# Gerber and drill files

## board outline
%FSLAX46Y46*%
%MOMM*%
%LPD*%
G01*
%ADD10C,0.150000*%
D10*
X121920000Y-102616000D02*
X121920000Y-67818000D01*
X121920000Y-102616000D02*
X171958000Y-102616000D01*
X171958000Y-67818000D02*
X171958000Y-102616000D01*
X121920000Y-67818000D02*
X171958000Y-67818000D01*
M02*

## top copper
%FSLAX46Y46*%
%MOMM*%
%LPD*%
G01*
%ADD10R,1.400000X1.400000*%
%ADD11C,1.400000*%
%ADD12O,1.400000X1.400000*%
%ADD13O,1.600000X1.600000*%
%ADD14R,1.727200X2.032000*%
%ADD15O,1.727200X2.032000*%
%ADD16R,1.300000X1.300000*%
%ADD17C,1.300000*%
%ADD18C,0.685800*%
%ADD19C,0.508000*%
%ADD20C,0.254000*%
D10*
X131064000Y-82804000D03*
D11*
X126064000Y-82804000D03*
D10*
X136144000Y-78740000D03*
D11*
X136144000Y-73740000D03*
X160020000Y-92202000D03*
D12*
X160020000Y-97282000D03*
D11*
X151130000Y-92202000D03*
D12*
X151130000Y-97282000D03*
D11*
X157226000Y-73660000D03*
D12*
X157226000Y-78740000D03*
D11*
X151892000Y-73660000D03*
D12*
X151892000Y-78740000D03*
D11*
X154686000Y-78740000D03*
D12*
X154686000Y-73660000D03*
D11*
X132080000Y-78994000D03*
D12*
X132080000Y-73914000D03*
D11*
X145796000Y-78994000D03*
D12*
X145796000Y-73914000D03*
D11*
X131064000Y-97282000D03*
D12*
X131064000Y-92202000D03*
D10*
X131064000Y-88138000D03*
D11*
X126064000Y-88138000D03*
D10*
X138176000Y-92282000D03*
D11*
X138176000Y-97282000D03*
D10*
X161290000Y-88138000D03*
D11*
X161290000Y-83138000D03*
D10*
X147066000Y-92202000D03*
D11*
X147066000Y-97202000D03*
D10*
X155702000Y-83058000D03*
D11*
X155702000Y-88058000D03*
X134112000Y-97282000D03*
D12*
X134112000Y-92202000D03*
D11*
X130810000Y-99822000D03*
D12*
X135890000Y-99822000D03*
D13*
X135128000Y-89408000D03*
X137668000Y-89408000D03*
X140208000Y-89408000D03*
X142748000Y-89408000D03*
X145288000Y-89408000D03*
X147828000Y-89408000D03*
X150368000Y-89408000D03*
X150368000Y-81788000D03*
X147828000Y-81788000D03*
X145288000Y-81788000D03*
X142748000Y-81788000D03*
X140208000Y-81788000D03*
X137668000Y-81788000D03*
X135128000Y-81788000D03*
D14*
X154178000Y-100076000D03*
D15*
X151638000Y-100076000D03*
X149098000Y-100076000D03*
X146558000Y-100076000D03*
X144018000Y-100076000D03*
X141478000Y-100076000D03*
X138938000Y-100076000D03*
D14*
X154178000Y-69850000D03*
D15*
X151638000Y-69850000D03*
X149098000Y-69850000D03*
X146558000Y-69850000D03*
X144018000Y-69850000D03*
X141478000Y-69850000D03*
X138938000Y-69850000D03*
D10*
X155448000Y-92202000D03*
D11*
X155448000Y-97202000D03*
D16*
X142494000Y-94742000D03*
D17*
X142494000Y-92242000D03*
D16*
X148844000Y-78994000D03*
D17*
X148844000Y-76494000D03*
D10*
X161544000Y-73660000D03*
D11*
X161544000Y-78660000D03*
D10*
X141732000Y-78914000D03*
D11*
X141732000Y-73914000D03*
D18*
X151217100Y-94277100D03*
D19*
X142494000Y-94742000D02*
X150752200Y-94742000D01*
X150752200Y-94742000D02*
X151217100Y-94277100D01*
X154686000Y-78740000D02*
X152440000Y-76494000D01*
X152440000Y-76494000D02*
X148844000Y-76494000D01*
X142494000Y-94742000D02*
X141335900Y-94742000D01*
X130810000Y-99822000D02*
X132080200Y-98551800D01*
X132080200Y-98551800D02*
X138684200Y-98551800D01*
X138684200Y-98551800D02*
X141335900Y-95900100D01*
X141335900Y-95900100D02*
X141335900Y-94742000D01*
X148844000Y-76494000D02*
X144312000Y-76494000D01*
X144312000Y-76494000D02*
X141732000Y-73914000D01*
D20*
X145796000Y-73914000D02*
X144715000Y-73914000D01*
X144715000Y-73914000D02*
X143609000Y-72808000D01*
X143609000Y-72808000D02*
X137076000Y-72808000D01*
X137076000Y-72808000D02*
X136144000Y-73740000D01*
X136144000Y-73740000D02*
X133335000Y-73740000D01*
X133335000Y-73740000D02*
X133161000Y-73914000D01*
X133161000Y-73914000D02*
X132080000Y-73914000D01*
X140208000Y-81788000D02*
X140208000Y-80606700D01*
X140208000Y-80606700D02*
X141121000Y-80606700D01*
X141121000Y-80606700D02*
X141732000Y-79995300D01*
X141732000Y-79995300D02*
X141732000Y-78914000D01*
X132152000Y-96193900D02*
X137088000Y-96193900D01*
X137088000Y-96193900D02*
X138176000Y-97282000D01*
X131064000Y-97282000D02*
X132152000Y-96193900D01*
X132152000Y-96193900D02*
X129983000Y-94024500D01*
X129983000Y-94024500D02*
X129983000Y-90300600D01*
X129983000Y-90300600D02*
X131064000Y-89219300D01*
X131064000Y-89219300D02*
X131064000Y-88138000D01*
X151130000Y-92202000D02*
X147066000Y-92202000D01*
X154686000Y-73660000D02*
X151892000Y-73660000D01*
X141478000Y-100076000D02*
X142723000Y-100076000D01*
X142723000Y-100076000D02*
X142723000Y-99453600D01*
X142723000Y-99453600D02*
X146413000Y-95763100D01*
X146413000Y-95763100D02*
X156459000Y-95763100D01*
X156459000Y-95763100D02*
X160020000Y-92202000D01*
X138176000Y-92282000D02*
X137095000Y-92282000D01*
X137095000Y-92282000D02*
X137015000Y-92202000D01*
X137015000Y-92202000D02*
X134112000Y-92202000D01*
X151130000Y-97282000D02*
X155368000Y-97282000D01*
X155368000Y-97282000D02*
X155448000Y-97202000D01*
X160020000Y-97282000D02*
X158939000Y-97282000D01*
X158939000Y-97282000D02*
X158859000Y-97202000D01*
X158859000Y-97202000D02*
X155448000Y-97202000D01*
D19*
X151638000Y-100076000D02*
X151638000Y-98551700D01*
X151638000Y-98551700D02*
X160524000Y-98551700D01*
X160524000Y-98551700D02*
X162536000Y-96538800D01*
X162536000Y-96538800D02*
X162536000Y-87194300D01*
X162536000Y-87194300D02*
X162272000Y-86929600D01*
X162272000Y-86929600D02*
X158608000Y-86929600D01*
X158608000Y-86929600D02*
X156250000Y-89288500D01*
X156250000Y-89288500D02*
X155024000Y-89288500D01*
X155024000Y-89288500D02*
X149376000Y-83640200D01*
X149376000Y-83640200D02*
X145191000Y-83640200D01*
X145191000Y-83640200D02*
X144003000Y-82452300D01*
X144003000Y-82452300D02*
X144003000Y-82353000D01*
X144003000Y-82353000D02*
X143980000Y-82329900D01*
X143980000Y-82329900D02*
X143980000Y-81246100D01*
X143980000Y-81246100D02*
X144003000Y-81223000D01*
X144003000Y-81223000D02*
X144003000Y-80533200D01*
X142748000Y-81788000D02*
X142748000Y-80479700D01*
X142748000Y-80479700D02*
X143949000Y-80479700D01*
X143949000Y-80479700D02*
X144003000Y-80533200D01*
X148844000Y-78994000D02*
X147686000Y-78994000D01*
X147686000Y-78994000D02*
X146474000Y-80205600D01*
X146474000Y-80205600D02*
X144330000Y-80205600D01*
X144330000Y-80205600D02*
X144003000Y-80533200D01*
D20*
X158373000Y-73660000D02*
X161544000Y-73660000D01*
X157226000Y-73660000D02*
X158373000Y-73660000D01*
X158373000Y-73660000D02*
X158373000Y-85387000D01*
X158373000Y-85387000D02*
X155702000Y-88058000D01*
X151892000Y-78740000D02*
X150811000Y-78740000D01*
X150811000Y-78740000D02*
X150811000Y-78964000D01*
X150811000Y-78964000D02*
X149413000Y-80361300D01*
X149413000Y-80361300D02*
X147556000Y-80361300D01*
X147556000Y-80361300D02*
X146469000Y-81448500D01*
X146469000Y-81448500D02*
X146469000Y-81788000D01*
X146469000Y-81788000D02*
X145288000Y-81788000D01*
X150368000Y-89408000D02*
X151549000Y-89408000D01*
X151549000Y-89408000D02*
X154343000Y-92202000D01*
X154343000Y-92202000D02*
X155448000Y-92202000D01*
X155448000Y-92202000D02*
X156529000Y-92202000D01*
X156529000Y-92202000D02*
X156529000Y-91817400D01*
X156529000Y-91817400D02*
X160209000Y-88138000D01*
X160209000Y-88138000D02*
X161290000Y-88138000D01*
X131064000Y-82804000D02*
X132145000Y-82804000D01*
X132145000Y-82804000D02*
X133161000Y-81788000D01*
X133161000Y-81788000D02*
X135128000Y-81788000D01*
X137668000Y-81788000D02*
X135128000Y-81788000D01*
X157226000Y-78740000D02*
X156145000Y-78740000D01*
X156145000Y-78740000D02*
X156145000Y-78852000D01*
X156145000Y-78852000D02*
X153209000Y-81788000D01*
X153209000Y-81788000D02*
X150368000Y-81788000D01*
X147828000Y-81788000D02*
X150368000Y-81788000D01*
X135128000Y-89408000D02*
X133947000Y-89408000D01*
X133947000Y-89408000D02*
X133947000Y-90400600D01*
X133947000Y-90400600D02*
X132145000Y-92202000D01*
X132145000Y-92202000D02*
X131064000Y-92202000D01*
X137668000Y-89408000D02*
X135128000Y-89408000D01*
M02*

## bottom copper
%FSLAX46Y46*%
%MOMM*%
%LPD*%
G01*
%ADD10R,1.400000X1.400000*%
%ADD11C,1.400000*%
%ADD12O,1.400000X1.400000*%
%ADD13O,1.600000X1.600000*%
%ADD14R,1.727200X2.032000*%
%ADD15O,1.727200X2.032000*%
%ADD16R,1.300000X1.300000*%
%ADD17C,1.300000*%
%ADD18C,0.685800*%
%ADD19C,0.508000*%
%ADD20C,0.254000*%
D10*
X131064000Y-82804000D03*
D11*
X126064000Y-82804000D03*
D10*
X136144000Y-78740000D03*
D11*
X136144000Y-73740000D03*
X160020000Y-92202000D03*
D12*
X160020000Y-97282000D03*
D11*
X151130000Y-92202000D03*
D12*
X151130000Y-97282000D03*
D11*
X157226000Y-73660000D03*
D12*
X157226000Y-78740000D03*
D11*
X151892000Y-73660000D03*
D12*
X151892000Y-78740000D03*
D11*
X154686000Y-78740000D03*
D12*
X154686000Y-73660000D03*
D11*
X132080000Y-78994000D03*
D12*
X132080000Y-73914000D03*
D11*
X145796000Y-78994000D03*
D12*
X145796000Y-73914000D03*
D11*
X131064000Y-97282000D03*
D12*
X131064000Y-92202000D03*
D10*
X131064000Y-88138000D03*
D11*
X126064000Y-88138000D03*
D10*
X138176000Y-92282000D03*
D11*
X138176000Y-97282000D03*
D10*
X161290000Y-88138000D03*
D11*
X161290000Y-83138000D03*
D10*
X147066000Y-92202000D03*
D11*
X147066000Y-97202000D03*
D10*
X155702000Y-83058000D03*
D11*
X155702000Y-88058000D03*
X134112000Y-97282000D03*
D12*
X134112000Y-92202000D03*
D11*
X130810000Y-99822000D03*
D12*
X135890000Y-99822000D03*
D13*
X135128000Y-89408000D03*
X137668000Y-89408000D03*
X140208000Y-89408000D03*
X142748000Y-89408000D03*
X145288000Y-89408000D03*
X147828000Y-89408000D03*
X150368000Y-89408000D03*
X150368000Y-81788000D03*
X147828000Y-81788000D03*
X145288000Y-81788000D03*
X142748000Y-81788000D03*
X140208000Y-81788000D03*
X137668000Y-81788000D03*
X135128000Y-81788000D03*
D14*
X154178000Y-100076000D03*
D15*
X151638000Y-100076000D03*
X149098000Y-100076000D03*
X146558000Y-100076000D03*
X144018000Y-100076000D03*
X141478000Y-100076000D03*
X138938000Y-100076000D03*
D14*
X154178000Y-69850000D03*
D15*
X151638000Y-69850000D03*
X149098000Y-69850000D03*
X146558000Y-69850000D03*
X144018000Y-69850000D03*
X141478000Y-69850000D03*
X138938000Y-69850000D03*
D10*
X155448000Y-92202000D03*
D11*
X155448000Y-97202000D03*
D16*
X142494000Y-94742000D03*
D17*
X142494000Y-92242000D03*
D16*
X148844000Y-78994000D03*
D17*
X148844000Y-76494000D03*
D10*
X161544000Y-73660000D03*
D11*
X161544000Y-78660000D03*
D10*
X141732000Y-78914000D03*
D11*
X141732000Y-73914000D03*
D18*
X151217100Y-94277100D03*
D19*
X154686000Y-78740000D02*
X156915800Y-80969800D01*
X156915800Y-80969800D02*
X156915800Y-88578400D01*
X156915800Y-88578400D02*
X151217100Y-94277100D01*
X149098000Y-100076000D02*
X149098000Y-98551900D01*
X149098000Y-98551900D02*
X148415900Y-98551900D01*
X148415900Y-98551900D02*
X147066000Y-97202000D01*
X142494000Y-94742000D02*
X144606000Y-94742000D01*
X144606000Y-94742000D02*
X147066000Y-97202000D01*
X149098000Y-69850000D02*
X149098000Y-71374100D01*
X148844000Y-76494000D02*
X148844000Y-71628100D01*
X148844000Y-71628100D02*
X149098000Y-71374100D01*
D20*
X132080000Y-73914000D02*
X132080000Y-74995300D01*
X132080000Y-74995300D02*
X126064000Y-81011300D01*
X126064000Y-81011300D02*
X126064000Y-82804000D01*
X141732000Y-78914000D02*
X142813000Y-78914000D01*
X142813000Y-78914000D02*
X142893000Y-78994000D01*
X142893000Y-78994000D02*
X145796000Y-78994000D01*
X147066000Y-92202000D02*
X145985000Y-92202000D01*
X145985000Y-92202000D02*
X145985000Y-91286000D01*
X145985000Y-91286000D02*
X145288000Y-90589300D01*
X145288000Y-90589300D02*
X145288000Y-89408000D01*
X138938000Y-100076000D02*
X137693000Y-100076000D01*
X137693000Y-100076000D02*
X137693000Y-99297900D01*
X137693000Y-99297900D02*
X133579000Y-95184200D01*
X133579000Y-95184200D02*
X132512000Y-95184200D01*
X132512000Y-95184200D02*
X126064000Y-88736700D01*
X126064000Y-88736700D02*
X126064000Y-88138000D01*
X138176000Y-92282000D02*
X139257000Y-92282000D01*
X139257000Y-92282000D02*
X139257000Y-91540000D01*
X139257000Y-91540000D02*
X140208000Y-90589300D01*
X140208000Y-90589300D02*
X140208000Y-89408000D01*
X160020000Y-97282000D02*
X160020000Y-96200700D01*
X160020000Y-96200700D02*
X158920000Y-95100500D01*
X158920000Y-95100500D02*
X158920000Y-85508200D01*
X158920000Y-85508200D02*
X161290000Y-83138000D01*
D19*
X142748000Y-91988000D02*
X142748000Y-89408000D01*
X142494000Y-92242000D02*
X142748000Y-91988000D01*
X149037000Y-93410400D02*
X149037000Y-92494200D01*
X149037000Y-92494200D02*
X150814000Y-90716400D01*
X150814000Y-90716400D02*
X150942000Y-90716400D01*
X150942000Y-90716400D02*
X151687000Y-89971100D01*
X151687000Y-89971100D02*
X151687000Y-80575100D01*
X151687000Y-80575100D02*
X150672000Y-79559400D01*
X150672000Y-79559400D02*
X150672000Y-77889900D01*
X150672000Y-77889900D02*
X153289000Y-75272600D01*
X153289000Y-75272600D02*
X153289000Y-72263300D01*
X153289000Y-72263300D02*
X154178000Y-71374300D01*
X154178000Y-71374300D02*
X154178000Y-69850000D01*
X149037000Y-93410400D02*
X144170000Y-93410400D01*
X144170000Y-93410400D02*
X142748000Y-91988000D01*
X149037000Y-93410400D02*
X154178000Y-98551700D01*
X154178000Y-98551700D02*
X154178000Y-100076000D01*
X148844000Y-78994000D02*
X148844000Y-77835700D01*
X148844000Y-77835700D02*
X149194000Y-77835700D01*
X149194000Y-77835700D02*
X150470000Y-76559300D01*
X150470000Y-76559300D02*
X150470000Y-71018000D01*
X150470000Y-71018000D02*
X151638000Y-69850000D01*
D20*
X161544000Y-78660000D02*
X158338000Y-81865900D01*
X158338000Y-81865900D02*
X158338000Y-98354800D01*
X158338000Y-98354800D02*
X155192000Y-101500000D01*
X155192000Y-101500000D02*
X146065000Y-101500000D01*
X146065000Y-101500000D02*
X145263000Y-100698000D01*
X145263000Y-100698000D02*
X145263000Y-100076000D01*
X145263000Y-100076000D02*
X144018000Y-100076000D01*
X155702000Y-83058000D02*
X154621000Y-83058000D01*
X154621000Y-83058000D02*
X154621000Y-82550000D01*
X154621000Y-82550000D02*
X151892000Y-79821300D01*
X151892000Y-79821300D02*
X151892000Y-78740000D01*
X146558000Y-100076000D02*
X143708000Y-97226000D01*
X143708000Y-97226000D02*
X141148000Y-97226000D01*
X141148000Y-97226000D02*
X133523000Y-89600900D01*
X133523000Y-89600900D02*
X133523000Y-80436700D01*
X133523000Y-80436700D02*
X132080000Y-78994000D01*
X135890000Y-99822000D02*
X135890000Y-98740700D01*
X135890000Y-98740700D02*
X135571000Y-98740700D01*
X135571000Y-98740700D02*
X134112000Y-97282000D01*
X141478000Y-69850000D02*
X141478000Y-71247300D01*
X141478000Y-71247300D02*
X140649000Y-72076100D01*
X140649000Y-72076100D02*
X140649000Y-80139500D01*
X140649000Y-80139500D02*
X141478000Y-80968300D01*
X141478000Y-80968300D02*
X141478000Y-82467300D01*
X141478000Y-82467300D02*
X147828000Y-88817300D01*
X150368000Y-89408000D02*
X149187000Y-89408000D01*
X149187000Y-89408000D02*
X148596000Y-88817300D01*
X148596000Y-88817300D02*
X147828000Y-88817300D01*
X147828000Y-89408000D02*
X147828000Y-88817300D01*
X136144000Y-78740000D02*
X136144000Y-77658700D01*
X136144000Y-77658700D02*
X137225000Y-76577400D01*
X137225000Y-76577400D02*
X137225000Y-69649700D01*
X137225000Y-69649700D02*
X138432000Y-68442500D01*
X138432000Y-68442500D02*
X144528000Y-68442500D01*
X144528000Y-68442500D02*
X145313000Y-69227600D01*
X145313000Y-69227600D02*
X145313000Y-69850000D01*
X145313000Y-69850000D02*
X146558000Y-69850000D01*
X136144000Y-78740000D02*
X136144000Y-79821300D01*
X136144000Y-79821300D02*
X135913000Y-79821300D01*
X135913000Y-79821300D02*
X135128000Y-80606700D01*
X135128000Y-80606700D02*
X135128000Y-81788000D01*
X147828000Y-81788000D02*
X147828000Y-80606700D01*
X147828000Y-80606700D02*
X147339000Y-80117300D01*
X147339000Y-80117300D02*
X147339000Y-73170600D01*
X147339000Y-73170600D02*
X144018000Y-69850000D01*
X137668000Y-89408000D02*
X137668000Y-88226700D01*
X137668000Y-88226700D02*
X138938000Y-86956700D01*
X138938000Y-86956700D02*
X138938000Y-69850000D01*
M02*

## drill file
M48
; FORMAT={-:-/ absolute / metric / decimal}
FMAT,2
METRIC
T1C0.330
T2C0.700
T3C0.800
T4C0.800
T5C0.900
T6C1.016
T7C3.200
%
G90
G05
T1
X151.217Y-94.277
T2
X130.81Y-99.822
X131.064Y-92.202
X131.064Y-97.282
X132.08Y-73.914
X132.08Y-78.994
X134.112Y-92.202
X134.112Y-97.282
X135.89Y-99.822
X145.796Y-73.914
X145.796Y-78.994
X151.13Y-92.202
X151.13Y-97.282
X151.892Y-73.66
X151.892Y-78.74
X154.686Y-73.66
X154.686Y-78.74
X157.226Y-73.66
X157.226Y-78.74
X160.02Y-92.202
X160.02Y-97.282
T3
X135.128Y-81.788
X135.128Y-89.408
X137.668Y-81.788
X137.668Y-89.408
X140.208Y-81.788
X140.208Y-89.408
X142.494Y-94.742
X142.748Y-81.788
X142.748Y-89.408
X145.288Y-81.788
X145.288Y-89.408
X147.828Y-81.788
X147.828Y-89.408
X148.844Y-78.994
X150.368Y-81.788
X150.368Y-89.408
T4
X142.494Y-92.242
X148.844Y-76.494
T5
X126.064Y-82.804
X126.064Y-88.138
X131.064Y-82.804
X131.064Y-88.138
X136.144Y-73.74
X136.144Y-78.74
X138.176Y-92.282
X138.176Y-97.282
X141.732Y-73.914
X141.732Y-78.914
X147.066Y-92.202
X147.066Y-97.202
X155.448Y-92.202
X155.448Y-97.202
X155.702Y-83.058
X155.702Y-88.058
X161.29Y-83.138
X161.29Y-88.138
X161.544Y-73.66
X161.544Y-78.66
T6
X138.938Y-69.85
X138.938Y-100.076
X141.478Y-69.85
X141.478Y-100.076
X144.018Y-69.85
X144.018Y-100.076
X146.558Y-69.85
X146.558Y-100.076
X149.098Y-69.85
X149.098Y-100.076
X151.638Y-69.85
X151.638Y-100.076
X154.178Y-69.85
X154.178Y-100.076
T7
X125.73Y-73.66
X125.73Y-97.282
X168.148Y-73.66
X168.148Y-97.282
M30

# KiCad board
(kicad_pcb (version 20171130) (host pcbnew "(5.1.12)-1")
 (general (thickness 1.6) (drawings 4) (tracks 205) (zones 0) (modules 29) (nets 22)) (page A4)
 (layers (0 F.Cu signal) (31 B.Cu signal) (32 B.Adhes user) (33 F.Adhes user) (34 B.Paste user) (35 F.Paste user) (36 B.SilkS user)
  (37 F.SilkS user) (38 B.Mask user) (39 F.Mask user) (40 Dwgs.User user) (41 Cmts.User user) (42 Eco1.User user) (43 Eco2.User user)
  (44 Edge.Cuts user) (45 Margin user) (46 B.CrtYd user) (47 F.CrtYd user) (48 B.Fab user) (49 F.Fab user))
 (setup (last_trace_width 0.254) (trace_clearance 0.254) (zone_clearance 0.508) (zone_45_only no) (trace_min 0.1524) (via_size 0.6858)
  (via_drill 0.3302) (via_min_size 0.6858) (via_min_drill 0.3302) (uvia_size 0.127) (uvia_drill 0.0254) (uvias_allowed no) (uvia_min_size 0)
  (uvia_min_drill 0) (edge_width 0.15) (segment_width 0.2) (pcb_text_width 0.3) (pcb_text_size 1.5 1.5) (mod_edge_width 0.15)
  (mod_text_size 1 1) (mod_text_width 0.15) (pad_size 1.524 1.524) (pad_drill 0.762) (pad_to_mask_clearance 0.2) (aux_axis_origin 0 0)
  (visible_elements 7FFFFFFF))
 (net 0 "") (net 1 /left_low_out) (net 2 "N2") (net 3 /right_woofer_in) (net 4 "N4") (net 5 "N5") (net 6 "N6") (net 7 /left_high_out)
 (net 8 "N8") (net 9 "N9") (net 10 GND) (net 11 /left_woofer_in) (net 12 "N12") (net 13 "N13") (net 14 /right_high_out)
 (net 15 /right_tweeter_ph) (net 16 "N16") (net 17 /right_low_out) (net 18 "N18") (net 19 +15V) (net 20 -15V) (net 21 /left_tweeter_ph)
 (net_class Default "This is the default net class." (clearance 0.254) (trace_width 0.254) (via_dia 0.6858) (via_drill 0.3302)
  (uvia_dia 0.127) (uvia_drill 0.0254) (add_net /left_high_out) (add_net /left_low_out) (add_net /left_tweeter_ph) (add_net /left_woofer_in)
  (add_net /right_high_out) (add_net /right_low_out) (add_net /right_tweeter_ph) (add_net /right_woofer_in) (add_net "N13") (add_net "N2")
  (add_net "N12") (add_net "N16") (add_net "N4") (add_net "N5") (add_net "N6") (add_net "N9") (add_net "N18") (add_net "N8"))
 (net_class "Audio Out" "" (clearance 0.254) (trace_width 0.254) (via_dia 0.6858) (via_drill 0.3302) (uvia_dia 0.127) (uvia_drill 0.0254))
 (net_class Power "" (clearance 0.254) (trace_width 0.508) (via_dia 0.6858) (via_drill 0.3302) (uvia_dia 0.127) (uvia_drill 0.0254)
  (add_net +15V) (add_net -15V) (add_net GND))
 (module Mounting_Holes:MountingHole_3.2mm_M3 (layer F.Cu) (at 125.73 97.282)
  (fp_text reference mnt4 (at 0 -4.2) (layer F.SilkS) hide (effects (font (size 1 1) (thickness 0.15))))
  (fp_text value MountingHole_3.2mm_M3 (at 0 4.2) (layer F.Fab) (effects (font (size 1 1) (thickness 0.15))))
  (pad 1 np_thru_hole circle (at 0 0) (size 3.2 3.2) (drill 3.2) (layers *.Cu *.Mask)))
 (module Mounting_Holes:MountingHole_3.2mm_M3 (layer F.Cu) (at 125.73 73.66)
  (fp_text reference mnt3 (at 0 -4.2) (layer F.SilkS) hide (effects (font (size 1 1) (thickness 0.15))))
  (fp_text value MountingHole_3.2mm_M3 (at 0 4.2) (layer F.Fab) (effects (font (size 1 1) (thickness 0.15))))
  (pad 1 np_thru_hole circle (at 0 0) (size 3.2 3.2) (drill 3.2) (layers *.Cu *.Mask)))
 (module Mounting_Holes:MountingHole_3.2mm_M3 (layer F.Cu) (at 168.148 97.282)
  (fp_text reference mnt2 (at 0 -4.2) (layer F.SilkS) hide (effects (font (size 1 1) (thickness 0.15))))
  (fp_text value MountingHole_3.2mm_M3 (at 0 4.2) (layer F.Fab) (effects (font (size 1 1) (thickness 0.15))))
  (pad 1 np_thru_hole circle (at 0 0) (size 3.2 3.2) (drill 3.2) (layers *.Cu *.Mask)))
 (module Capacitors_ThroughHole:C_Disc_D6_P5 (layer F.Cu) (at 131.064 82.804 180)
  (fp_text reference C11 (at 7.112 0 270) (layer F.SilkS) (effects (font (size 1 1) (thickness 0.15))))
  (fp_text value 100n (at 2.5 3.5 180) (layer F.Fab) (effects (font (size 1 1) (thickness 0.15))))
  (pad 1 thru_hole rect (at 0 0 180) (size 1.4 1.4) (drill 0.9) (layers *.Cu *.Mask) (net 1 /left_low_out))
  (pad 2 thru_hole circle (at 5 0 180) (size 1.4 1.4) (drill 0.9) (layers *.Cu *.Mask) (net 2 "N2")))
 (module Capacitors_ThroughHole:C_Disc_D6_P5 (layer F.Cu) (at 136.144 78.74 90)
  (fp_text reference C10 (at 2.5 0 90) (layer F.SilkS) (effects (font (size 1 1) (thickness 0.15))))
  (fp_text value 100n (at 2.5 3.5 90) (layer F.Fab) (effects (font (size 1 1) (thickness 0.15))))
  (pad 1 thru_hole rect (at 0 0 90) (size 1.4 1.4) (drill 0.9) (layers *.Cu *.Mask) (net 1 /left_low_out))
  (pad 2 thru_hole circle (at 5 0 90) (size 1.4 1.4) (drill 0.9) (layers *.Cu *.Mask) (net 2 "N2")))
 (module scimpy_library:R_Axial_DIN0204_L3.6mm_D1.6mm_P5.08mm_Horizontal (layer F.Cu) (at 160.02 92.202 270)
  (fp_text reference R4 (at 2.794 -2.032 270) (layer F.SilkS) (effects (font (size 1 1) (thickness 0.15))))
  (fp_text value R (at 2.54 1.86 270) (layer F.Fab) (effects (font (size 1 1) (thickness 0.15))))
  (pad 1 thru_hole circle (at 0 0 270) (size 1.4 1.4) (drill 0.7) (layers *.Cu *.Mask) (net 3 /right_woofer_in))
  (pad 2 thru_hole oval (at 5.08 0 270) (size 1.4 1.4) (drill 0.7) (layers *.Cu *.Mask) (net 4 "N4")))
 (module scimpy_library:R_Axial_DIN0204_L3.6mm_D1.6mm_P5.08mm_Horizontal (layer F.Cu) (at 151.13 92.202 270)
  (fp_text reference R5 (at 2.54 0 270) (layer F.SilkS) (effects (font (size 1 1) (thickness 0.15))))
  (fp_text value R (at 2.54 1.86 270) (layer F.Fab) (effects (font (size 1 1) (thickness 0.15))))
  (pad 1 thru_hole circle (at 0 0 270) (size 1.4 1.4) (drill 0.7) (layers *.Cu *.Mask) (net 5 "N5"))
  (pad 2 thru_hole oval (at 5.08 0 270) (size 1.4 1.4) (drill 0.7) (layers *.Cu *.Mask) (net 4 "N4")))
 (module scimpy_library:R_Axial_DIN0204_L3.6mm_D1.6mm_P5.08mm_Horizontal (layer F.Cu) (at 157.226 73.66 270)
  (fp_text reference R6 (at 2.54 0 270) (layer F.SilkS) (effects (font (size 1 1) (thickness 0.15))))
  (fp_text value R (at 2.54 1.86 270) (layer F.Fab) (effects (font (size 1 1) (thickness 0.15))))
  (pad 1 thru_hole circle (at 0 0 270) (size 1.4 1.4) (drill 0.7) (layers *.Cu *.Mask) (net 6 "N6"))
  (pad 2 thru_hole oval (at 5.08 0 270) (size 1.4 1.4) (drill 0.7) (layers *.Cu *.Mask) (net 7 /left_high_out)))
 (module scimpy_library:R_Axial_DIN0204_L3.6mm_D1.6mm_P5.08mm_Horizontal (layer F.Cu) (at 151.892 73.66 270)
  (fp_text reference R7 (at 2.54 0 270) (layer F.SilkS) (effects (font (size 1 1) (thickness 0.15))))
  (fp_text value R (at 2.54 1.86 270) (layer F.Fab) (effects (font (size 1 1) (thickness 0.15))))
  (pad 1 thru_hole circle (at 0 0 270) (size 1.4 1.4) (drill 0.7) (layers *.Cu *.Mask) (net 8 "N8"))
  (pad 2 thru_hole oval (at 5.08 0 270) (size 1.4 1.4) (drill 0.7) (layers *.Cu *.Mask) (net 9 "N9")))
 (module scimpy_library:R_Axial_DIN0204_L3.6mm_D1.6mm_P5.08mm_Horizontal (layer F.Cu) (at 154.686 78.74 90)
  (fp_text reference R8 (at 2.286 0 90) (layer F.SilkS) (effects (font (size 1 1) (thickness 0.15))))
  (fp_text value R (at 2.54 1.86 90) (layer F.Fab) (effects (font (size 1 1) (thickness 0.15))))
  (pad 1 thru_hole circle (at 0 0 90) (size 1.4 1.4) (drill 0.7) (layers *.Cu *.Mask) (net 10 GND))
  (pad 2 thru_hole oval (at 5.08 0 90) (size 1.4 1.4) (drill 0.7) (layers *.Cu *.Mask) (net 8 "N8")))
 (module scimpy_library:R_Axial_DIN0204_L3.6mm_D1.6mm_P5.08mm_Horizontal (layer F.Cu) (at 132.08 78.994 90)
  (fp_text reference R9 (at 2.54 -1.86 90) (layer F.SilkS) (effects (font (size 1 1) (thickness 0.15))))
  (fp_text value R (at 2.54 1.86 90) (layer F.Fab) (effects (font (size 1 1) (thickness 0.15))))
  (pad 1 thru_hole circle (at 0 0 90) (size 1.4 1.4) (drill 0.7) (layers *.Cu *.Mask) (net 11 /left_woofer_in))
  (pad 2 thru_hole oval (at 5.08 0 90) (size 1.4 1.4) (drill 0.7) (layers *.Cu *.Mask) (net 2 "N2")))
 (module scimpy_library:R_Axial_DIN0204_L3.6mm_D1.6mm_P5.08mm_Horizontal (layer F.Cu) (at 145.796 78.994 90)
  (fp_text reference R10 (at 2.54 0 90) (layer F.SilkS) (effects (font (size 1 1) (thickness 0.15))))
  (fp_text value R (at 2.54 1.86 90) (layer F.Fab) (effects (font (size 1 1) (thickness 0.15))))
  (pad 1 thru_hole circle (at 0 0 90) (size 1.4 1.4) (drill 0.7) (layers *.Cu *.Mask) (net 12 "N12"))
  (pad 2 thru_hole oval (at 5.08 0 90) (size 1.4 1.4) (drill 0.7) (layers *.Cu *.Mask) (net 2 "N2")))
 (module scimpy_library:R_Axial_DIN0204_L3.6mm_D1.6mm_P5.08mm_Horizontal (layer F.Cu) (at 131.064 97.282 90)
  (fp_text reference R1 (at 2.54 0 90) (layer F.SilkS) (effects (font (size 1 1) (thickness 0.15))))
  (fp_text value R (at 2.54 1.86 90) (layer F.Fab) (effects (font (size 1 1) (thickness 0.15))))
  (pad 1 thru_hole circle (at 0 0 90) (size 1.4 1.4) (drill 0.7) (layers *.Cu *.Mask) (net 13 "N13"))
  (pad 2 thru_hole oval (at 5.08 0 90) (size 1.4 1.4) (drill 0.7) (layers *.Cu *.Mask) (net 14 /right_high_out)))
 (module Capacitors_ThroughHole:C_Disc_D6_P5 (layer F.Cu) (at 131.064 88.138 180)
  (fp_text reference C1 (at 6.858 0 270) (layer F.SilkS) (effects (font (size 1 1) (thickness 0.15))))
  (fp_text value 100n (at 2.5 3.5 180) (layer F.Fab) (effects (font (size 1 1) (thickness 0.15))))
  (pad 1 thru_hole rect (at 0 0 180) (size 1.4 1.4) (drill 0.9) (layers *.Cu *.Mask) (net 13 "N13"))
  (pad 2 thru_hole circle (at 5 0 180) (size 1.4 1.4) (drill 0.9) (layers *.Cu *.Mask) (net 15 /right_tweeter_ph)))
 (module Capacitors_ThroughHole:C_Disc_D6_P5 (layer F.Cu) (at 138.176 92.282 270)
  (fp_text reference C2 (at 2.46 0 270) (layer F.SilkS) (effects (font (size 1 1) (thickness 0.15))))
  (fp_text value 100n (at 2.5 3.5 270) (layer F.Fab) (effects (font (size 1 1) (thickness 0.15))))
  (pad 1 thru_hole rect (at 0 0 270) (size 1.4 1.4) (drill 0.9) (layers *.Cu *.Mask) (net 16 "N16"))
  (pad 2 thru_hole circle (at 5 0 270) (size 1.4 1.4) (drill 0.9) (layers *.Cu *.Mask) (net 13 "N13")))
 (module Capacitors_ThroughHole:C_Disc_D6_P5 (layer F.Cu) (at 161.29 88.138 90)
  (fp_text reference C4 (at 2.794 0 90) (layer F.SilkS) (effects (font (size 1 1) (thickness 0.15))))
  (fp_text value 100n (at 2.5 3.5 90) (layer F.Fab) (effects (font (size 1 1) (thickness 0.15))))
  (pad 1 thru_hole rect (at 0 0 90) (size 1.4 1.4) (drill 0.9) (layers *.Cu *.Mask) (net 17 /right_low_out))
  (pad 2 thru_hole circle (at 5 0 90) (size 1.4 1.4) (drill 0.9) (layers *.Cu *.Mask) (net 4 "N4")))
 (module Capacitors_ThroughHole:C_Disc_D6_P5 (layer F.Cu) (at 147.066 92.202 270)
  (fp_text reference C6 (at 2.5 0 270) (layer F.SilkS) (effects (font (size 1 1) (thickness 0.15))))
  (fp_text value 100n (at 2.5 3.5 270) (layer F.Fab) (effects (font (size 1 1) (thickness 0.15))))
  (pad 1 thru_hole rect (at 0 0 270) (size 1.4 1.4) (drill 0.9) (layers *.Cu *.Mask) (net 5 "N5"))
  (pad 2 thru_hole circle (at 5 0 270) (size 1.4 1.4) (drill 0.9) (layers *.Cu *.Mask) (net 10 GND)))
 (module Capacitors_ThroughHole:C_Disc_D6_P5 (layer F.Cu) (at 155.702 83.058 270)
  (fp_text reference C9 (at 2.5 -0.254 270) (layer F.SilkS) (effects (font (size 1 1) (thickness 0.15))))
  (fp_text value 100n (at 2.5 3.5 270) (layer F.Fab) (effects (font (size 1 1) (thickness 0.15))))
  (pad 1 thru_hole rect (at 0 0 270) (size 1.4 1.4) (drill 0.9) (layers *.Cu *.Mask) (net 9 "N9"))
  (pad 2 thru_hole circle (at 5 0 270) (size 1.4 1.4) (drill 0.9) (layers *.Cu *.Mask) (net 6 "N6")))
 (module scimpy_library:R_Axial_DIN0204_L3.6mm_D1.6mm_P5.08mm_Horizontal (layer F.Cu) (at 134.112 97.282 90)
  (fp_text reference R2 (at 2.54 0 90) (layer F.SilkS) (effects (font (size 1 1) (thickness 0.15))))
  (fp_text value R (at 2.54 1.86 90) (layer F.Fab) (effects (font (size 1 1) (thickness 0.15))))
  (pad 1 thru_hole circle (at 0 0 90) (size 1.4 1.4) (drill 0.7) (layers *.Cu *.Mask) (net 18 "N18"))
  (pad 2 thru_hole oval (at 5.08 0 90) (size 1.4 1.4) (drill 0.7) (layers *.Cu *.Mask) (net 16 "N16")))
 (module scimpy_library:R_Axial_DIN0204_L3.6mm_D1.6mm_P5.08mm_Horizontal (layer F.Cu) (at 130.81 99.822)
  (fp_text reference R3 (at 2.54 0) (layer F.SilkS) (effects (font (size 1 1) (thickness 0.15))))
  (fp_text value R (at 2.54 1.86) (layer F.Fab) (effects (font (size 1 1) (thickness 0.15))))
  (pad 1 thru_hole circle (at 0 0) (size 1.4 1.4) (drill 0.7) (layers *.Cu *.Mask) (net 10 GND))
  (pad 2 thru_hole oval (at 5.08 0) (size 1.4 1.4) (drill 0.7) (layers *.Cu *.Mask) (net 18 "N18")))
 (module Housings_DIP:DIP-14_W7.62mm (layer F.Cu) (at 135.128 89.408 90)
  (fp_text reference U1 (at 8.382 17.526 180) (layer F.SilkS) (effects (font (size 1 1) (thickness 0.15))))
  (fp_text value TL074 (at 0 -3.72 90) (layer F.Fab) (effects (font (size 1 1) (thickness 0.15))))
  (pad 1 thru_hole oval (at 0 0 90) (size 1.6 1.6) (drill 0.8) (layers *.Cu *.Mask) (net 14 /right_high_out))
  (pad 2 thru_hole oval (at 0 2.54 90) (size 1.6 1.6) (drill 0.8) (layers *.Cu *.Mask) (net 14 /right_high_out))
  (pad 3 thru_hole oval (at 0 5.08 90) (size 1.6 1.6) (drill 0.8) (layers *.Cu *.Mask) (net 16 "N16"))
  (pad 4 thru_hole oval (at 0 7.62 90) (size 1.6 1.6) (drill 0.8) (layers *.Cu *.Mask) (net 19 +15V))
  (pad 5 thru_hole oval (at 0 10.16 90) (size 1.6 1.6) (drill 0.8) (layers *.Cu *.Mask) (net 5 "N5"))
  (pad 6 thru_hole oval (at 0 12.7 90) (size 1.6 1.6) (drill 0.8) (layers *.Cu *.Mask) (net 17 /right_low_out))
  (pad 7 thru_hole oval (at 0 15.24 90) (size 1.6 1.6) (drill 0.8) (layers *.Cu *.Mask) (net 17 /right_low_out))
  (pad 8 thru_hole oval (at 7.62 15.24 90) (size 1.6 1.6) (drill 0.8) (layers *.Cu *.Mask) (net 7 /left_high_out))
  (pad 9 thru_hole oval (at 7.62 12.7 90) (size 1.6 1.6) (drill 0.8) (layers *.Cu *.Mask) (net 7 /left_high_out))
  (pad 10 thru_hole oval (at 7.62 10.16 90) (size 1.6 1.6) (drill 0.8) (layers *.Cu *.Mask) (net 9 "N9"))
  (pad 11 thru_hole oval (at 7.62 7.62 90) (size 1.6 1.6) (drill 0.8) (layers *.Cu *.Mask) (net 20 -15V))
  (pad 12 thru_hole oval (at 7.62 5.08 90) (size 1.6 1.6) (drill 0.8) (layers *.Cu *.Mask) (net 12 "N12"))
  (pad 13 thru_hole oval (at 7.62 2.54 90) (size 1.6 1.6) (drill 0.8) (layers *.Cu *.Mask) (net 1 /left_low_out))
  (pad 14 thru_hole oval (at 7.62 0 90) (size 1.6 1.6) (drill 0.8) (layers *.Cu *.Mask) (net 1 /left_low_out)))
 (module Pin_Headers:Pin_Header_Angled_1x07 (layer F.Cu) (at 154.178 100.076 270)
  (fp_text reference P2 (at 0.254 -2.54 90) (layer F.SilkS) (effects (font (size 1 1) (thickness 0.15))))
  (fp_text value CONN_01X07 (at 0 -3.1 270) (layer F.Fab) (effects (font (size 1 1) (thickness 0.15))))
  (pad 1 thru_hole rect (at 0 0 270) (size 2.032 1.7272) (drill 1.016) (layers *.Cu *.Mask) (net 19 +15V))
  (pad 2 thru_hole oval (at 0 2.54 270) (size 2.032 1.7272) (drill 1.016) (layers *.Cu *.Mask) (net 20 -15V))
  (pad 3 thru_hole oval (at 0 5.08 270) (size 2.032 1.7272) (drill 1.016) (layers *.Cu *.Mask) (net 10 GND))
  (pad 4 thru_hole oval (at 0 7.62 270) (size 2.032 1.7272) (drill 1.016) (layers *.Cu *.Mask) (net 11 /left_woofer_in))
  (pad 5 thru_hole oval (at 0 10.16 270) (size 2.032 1.7272) (drill 1.016) (layers *.Cu *.Mask) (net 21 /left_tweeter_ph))
  (pad 6 thru_hole oval (at 0 12.7 270) (size 2.032 1.7272) (drill 1.016) (layers *.Cu *.Mask) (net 3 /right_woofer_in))
  (pad 7 thru_hole oval (at 0 15.24 270) (size 2.032 1.7272) (drill 1.016) (layers *.Cu *.Mask) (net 15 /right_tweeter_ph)))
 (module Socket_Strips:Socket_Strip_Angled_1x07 (layer F.Cu) (at 154.178 69.85 180)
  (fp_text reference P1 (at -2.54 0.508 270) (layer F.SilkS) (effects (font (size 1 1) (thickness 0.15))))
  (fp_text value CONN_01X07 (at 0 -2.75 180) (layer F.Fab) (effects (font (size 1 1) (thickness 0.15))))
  (pad 1 thru_hole rect (at 0 0 180) (size 1.7272 2.032) (drill 1.016) (layers *.Cu *.Mask) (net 19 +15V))
  (pad 2 thru_hole oval (at 2.54 0 180) (size 1.7272 2.032) (drill 1.016) (layers *.Cu *.Mask) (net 20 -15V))
  (pad 3 thru_hole oval (at 5.08 0 180) (size 1.7272 2.032) (drill 1.016) (layers *.Cu *.Mask) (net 10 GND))
  (pad 4 thru_hole oval (at 7.62 0 180) (size 1.7272 2.032) (drill 1.016) (layers *.Cu *.Mask) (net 1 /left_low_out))
  (pad 5 thru_hole oval (at 10.16 0 180) (size 1.7272 2.032) (drill 1.016) (layers *.Cu *.Mask) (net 7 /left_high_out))
  (pad 6 thru_hole oval (at 12.7 0 180) (size 1.7272 2.032) (drill 1.016) (layers *.Cu *.Mask) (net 17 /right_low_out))
  (pad 7 thru_hole oval (at 15.24 0 180) (size 1.7272 2.032) (drill 1.016) (layers *.Cu *.Mask) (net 14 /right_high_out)))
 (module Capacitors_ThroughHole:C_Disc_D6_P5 (layer F.Cu) (at 155.448 92.202 270)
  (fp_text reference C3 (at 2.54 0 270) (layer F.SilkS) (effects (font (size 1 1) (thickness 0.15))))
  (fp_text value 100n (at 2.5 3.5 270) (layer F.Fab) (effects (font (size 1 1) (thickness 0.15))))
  (pad 1 thru_hole rect (at 0 0 270) (size 1.4 1.4) (drill 0.9) (layers *.Cu *.Mask) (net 17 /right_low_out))
  (pad 2 thru_hole circle (at 5 0 270) (size 1.4 1.4) (drill 0.9) (layers *.Cu *.Mask) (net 4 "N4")))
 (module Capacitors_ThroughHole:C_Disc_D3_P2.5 (layer F.Cu) (at 142.494 94.742 90)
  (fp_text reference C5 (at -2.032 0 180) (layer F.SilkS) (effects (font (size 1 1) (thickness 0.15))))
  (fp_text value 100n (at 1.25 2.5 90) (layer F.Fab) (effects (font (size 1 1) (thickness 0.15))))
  (pad 1 thru_hole rect (at 0 0 90) (size 1.3 1.3) (drill 0.8) (layers *.Cu *.Mask) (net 10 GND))
  (pad 2 thru_hole circle (at 2.5 0 90) (size 1.3 1.3) (drill 0.8001) (layers *.Cu *.Mask) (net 19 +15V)))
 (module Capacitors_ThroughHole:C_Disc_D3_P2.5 (layer F.Cu) (at 148.844 78.994 90)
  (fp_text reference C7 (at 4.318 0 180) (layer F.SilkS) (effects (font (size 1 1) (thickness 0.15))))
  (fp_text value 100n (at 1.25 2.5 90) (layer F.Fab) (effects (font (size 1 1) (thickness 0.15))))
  (pad 1 thru_hole rect (at 0 0 90) (size 1.3 1.3) (drill 0.8) (layers *.Cu *.Mask) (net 20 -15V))
  (pad 2 thru_hole circle (at 2.5 0 90) (size 1.3 1.3) (drill 0.8001) (layers *.Cu *.Mask) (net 10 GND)))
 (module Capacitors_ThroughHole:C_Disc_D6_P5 (layer F.Cu) (at 161.544 73.66 270)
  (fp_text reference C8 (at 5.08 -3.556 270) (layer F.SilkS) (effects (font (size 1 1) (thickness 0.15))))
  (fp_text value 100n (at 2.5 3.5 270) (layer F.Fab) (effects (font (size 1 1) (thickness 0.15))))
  (pad 1 thru_hole rect (at 0 0 270) (size 1.4 1.4) (drill 0.9) (layers *.Cu *.Mask) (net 6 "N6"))
  (pad 2 thru_hole circle (at 5 0 270) (size 1.4 1.4) (drill 0.9) (layers *.Cu *.Mask) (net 21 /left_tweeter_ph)))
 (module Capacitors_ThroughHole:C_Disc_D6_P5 (layer F.Cu) (at 141.732 78.914 90)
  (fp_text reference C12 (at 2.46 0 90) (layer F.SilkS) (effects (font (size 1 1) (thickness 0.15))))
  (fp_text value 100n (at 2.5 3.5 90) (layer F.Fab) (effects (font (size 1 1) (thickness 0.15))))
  (pad 1 thru_hole rect (at 0 0 90) (size 1.4 1.4) (drill 0.9) (layers *.Cu *.Mask) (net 12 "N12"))
  (pad 2 thru_hole circle (at 5 0 90) (size 1.4 1.4) (drill 0.9) (layers *.Cu *.Mask) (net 10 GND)))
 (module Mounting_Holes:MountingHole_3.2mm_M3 (layer F.Cu) (at 168.148 73.66)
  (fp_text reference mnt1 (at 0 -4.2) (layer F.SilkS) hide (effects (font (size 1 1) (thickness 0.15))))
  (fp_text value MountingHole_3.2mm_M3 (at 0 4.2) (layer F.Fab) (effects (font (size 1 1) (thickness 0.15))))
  (pad 1 np_thru_hole circle (at 0 0) (size 3.2 3.2) (drill 3.2) (layers *.Cu *.Mask)))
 (gr_line (start 121.92 102.616) (end 121.92 67.818) (angle 90) (layer Edge.Cuts) (width 0.15))
 (gr_line (start 121.92 102.616) (end 171.958 102.616) (angle 90) (layer Edge.Cuts) (width 0.15))
 (gr_line (start 171.958 67.818) (end 171.958 102.616) (angle 90) (layer Edge.Cuts) (width 0.15))
 (gr_line (start 121.92 67.818) (end 171.958 67.818) (angle 90) (layer Edge.Cuts) (width 0.15))
 (segment (start 142.494 94.742) (end 150.7522 94.742) (width 0.508) (layer F.Cu) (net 10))
 (segment (start 150.7522 94.742) (end 151.2171 94.2771) (width 0.508) (layer F.Cu) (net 10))
 (segment (start 154.686 78.74) (end 156.9158 80.9698) (width 0.508) (layer B.Cu) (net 10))
 (segment (start 156.9158 80.9698) (end 156.9158 88.5784) (width 0.508) (layer B.Cu) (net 10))
 (segment (start 156.9158 88.5784) (end 151.2171 94.2771) (width 0.508) (layer B.Cu) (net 10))
 (segment (start 154.686 78.74) (end 152.44 76.494) (width 0.508) (layer F.Cu) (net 10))
 (segment (start 152.44 76.494) (end 148.844 76.494) (width 0.508) (layer F.Cu) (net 10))
 (segment (start 142.494 94.742) (end 141.3359 94.742) (width 0.508) (layer F.Cu) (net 10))
 (segment (start 130.81 99.822) (end 132.0802 98.5518) (width 0.508) (layer F.Cu) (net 10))
 (segment (start 132.0802 98.5518) (end 138.6842 98.5518) (width 0.508) (layer F.Cu) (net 10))
 (segment (start 138.6842 98.5518) (end 141.3359 95.9001) (width 0.508) (layer F.Cu) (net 10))
 (segment (start 141.3359 95.9001) (end 141.3359 94.742) (width 0.508) (layer F.Cu) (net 10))
 (segment (start 149.098 100.076) (end 149.098 98.5519) (width 0.508) (layer B.Cu) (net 10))
 (segment (start 149.098 98.5519) (end 148.4159 98.5519) (width 0.508) (layer B.Cu) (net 10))
 (segment (start 148.4159 98.5519) (end 147.066 97.202) (width 0.508) (layer B.Cu) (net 10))
 (segment (start 148.844 76.494) (end 144.312 76.494) (width 0.508) (layer F.Cu) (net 10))
 (segment (start 144.312 76.494) (end 141.732 73.914) (width 0.508) (layer F.Cu) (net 10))
 (segment (start 142.494 94.742) (end 144.606 94.742) (width 0.508) (layer B.Cu) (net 10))
 (segment (start 144.606 94.742) (end 147.066 97.202) (width 0.508) (layer B.Cu) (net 10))
 (segment (start 149.098 69.85) (end 149.098 71.3741) (width 0.508) (layer B.Cu) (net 10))
 (segment (start 148.844 76.494) (end 148.844 71.6281) (width 0.508) (layer B.Cu) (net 10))
 (segment (start 148.844 71.6281) (end 149.098 71.3741) (width 0.508) (layer B.Cu) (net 10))
 (via (at 151.2171 94.2771) (size 0.6858) (layers F.Cu B.Cu) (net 10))
 (segment (start 145.796 73.914) (end 144.715 73.914) (width 0.254) (layer F.Cu) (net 2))
 (segment (start 144.715 73.914) (end 143.609 72.808) (width 0.254) (layer F.Cu) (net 2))
 (segment (start 143.609 72.808) (end 137.076 72.808) (width 0.254) (layer F.Cu) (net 2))
 (segment (start 137.076 72.808) (end 136.144 73.74) (width 0.254) (layer F.Cu) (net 2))
 (segment (start 136.144 73.74) (end 133.335 73.74) (width 0.254) (layer F.Cu) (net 2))
 (segment (start 133.335 73.74) (end 133.161 73.914) (width 0.254) (layer F.Cu) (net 2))
 (segment (start 133.161 73.914) (end 132.08 73.914) (width 0.254) (layer F.Cu) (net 2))
 (segment (start 132.08 73.914) (end 132.08 74.9953) (width 0.254) (layer B.Cu) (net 2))
 (segment (start 132.08 74.9953) (end 126.064 81.0113) (width 0.254) (layer B.Cu) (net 2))
 (segment (start 126.064 81.0113) (end 126.064 82.804) (width 0.254) (layer B.Cu) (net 2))
 (segment (start 140.208 81.788) (end 140.208 80.6067) (width 0.254) (layer F.Cu) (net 12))
 (segment (start 140.208 80.6067) (end 141.121 80.6067) (width 0.254) (layer F.Cu) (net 12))
 (segment (start 141.121 80.6067) (end 141.732 79.9953) (width 0.254) (layer F.Cu) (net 12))
 (segment (start 141.732 79.9953) (end 141.732 78.914) (width 0.254) (layer F.Cu) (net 12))
 (segment (start 141.732 78.914) (end 142.813 78.914) (width 0.254) (layer B.Cu) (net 12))
 (segment (start 142.813 78.914) (end 142.893 78.994) (width 0.254) (layer B.Cu) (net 12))
 (segment (start 142.893 78.994) (end 145.796 78.994) (width 0.254) (layer B.Cu) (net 12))
 (segment (start 132.152 96.1939) (end 137.088 96.1939) (width 0.254) (layer F.Cu) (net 13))
 (segment (start 137.088 96.1939) (end 138.176 97.282) (width 0.254) (layer F.Cu) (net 13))
 (segment (start 131.064 97.282) (end 132.152 96.1939) (width 0.254) (layer F.Cu) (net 13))
 (segment (start 132.152 96.1939) (end 129.983 94.0245) (width 0.254) (layer F.Cu) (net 13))
 (segment (start 129.983 94.0245) (end 129.983 90.3006) (width 0.254) (layer F.Cu) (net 13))
 (segment (start 129.983 90.3006) (end 131.064 89.2193) (width 0.254) (layer F.Cu) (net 13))
 (segment (start 131.064 89.2193) (end 131.064 88.138) (width 0.254) (layer F.Cu) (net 13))
 (segment (start 151.13 92.202) (end 147.066 92.202) (width 0.254) (layer F.Cu) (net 5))
 (segment (start 147.066 92.202) (end 145.985 92.202) (width 0.254) (layer B.Cu) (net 5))
 (segment (start 145.985 92.202) (end 145.985 91.286) (width 0.254) (layer B.Cu) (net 5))
 (segment (start 145.985 91.286) (end 145.288 90.5893) (width 0.254) (layer B.Cu) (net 5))
 (segment (start 145.288 90.5893) (end 145.288 89.408) (width 0.254) (layer B.Cu) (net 5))
 (segment (start 154.686 73.66) (end 151.892 73.66) (width 0.254) (layer F.Cu) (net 8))
 (segment (start 138.938 100.076) (end 137.693 100.076) (width 0.254) (layer B.Cu) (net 15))
 (segment (start 137.693 100.076) (end 137.693 99.2979) (width 0.254) (layer B.Cu) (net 15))
 (segment (start 137.693 99.2979) (end 133.579 95.1842) (width 0.254) (layer B.Cu) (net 15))
 (segment (start 133.579 95.1842) (end 132.512 95.1842) (width 0.254) (layer B.Cu) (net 15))
 (segment (start 132.512 95.1842) (end 126.064 88.7367) (width 0.254) (layer B.Cu) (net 15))
 (segment (start 126.064 88.7367) (end 126.064 88.138) (width 0.254) (layer B.Cu) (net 15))
 (segment (start 141.478 100.076) (end 142.723 100.076) (width 0.254) (layer F.Cu) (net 3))
 (segment (start 142.723 100.076) (end 142.723 99.4536) (width 0.254) (layer F.Cu) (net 3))
 (segment (start 142.723 99.4536) (end 146.413 95.7631) (width 0.254) (layer F.Cu) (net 3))
 (segment (start 146.413 95.7631) (end 156.459 95.7631) (width 0.254) (layer F.Cu) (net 3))
 (segment (start 156.459 95.7631) (end 160.02 92.202) (width 0.254) (layer F.Cu) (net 3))
 (segment (start 138.176 92.282) (end 139.257 92.282) (width 0.254) (layer B.Cu) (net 16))
 (segment (start 139.257 92.282) (end 139.257 91.54) (width 0.254) (layer B.Cu) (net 16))
 (segment (start 139.257 91.54) (end 140.208 90.5893) (width 0.254) (layer B.Cu) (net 16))
 (segment (start 140.208 90.5893) (end 140.208 89.408) (width 0.254) (layer B.Cu) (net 16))
 (segment (start 138.176 92.282) (end 137.095 92.282) (width 0.254) (layer F.Cu) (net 16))
 (segment (start 137.095 92.282) (end 137.015 92.202) (width 0.254) (layer F.Cu) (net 16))
 (segment (start 137.015 92.202) (end 134.112 92.202) (width 0.254) (layer F.Cu) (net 16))
 (segment (start 160.02 97.282) (end 160.02 96.2007) (width 0.254) (layer B.Cu) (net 4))
 (segment (start 160.02 96.2007) (end 158.92 95.1005) (width 0.254) (layer B.Cu) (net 4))
 (segment (start 158.92 95.1005) (end 158.92 85.5082) (width 0.254) (layer B.Cu) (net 4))
 (segment (start 158.92 85.5082) (end 161.29 83.138) (width 0.254) (layer B.Cu) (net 4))
 (segment (start 151.13 97.282) (end 155.368 97.282) (width 0.254) (layer F.Cu) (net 4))
 (segment (start 155.368 97.282) (end 155.448 97.202) (width 0.254) (layer F.Cu) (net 4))
 (segment (start 160.02 97.282) (end 158.939 97.282) (width 0.254) (layer F.Cu) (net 4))
 (segment (start 158.939 97.282) (end 158.859 97.202) (width 0.254) (layer F.Cu) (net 4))
 (segment (start 158.859 97.202) (end 155.448 97.202) (width 0.254) (layer F.Cu) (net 4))
 (segment (start 142.748 91.988) (end 142.748 89.408) (width 0.508) (layer B.Cu) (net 19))
 (segment (start 142.494 92.242) (end 142.748 91.988) (width 0.508) (layer B.Cu) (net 19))
 (segment (start 149.037 93.4104) (end 149.037 92.4942) (width 0.508) (layer B.Cu) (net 19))
 (segment (start 149.037 92.4942) (end 150.814 90.7164) (width 0.508) (layer B.Cu) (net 19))
 (segment (start 150.814 90.7164) (end 150.942 90.7164) (width 0.508) (layer B.Cu) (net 19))
 (segment (start 150.942 90.7164) (end 151.687 89.9711) (width 0.508) (layer B.Cu) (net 19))
 (segment (start 151.687 89.9711) (end 151.687 80.5751) (width 0.508) (layer B.Cu) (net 19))
 (segment (start 151.687 80.5751) (end 150.672 79.5594) (width 0.508) (layer B.Cu) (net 19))
 (segment (start 150.672 79.5594) (end 150.672 77.8899) (width 0.508) (layer B.Cu) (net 19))
 (segment (start 150.672 77.8899) (end 153.289 75.2726) (width 0.508) (layer B.Cu) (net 19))
 (segment (start 153.289 75.2726) (end 153.289 72.2633) (width 0.508) (layer B.Cu) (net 19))
 (segment (start 153.289 72.2633) (end 154.178 71.3743) (width 0.508) (layer B.Cu) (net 19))
 (segment (start 154.178 71.3743) (end 154.178 69.85) (width 0.508) (layer B.Cu) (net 19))
 (segment (start 149.037 93.4104) (end 144.17 93.4104) (width 0.508) (layer B.Cu) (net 19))
 (segment (start 144.17 93.4104) (end 142.748 91.988) (width 0.508) (layer B.Cu) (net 19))
 (segment (start 149.037 93.4104) (end 154.178 98.5517) (width 0.508) (layer B.Cu) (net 19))
 (segment (start 154.178 98.5517) (end 154.178 100.076) (width 0.508) (layer B.Cu) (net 19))
 (segment (start 148.844 78.994) (end 148.844 77.8357) (width 0.508) (layer B.Cu) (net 20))
 (segment (start 148.844 77.8357) (end 149.194 77.8357) (width 0.508) (layer B.Cu) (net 20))
 (segment (start 149.194 77.8357) (end 150.47 76.5593) (width 0.508) (layer B.Cu) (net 20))
 (segment (start 150.47 76.5593) (end 150.47 71.018) (width 0.508) (layer B.Cu) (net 20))
 (segment (start 150.47 71.018) (end 151.638 69.85) (width 0.508) (layer B.Cu) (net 20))
 (segment (start 151.638 100.076) (end 151.638 98.5517) (width 0.508) (layer F.Cu) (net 20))
 (segment (start 151.638 98.5517) (end 160.524 98.5517) (width 0.508) (layer F.Cu) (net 20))
 (segment (start 160.524 98.5517) (end 162.536 96.5388) (width 0.508) (layer F.Cu) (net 20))
 (segment (start 162.536 96.5388) (end 162.536 87.1943) (width 0.508) (layer F.Cu) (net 20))
 (segment (start 162.536 87.1943) (end 162.272 86.9296) (width 0.508) (layer F.Cu) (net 20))
 (segment (start 162.272 86.9296) (end 158.608 86.9296) (width 0.508) (layer F.Cu) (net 20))
 (segment (start 158.608 86.9296) (end 156.25 89.2885) (width 0.508) (layer F.Cu) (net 20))
 (segment (start 156.25 89.2885) (end 155.024 89.2885) (width 0.508) (layer F.Cu) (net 20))
 (segment (start 155.024 89.2885) (end 149.376 83.6402) (width 0.508) (layer F.Cu) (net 20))
 (segment (start 149.376 83.6402) (end 145.191 83.6402) (width 0.508) (layer F.Cu) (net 20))
 (segment (start 145.191 83.6402) (end 144.003 82.4523) (width 0.508) (layer F.Cu) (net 20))
 (segment (start 144.003 82.4523) (end 144.003 82.353) (width 0.508) (layer F.Cu) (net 20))
 (segment (start 144.003 82.353) (end 143.98 82.3299) (width 0.508) (layer F.Cu) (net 20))
 (segment (start 143.98 82.3299) (end 143.98 81.2461) (width 0.508) (layer F.Cu) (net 20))
 (segment (start 143.98 81.2461) (end 144.003 81.223) (width 0.508) (layer F.Cu) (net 20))
 (segment (start 144.003 81.223) (end 144.003 80.5332) (width 0.508) (layer F.Cu) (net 20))
 (segment (start 142.748 81.788) (end 142.748 80.4797) (width 0.508) (layer F.Cu) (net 20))
 (segment (start 142.748 80.4797) (end 143.949 80.4797) (width 0.508) (layer F.Cu) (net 20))
 (segment (start 143.949 80.4797) (end 144.003 80.5332) (width 0.508) (layer F.Cu) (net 20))
 (segment (start 148.844 78.994) (end 147.686 78.994) (width 0.508) (layer F.Cu) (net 20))
 (segment (start 147.686 78.994) (end 146.474 80.2056) (width 0.508) (layer F.Cu) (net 20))
 (segment (start 146.474 80.2056) (end 144.33 80.2056) (width 0.508) (layer F.Cu) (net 20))
 (segment (start 144.33 80.2056) (end 144.003 80.5332) (width 0.508) (layer F.Cu) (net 20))
 (segment (start 158.373 73.66) (end 161.544 73.66) (width 0.254) (layer F.Cu) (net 6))
 (segment (start 157.226 73.66) (end 158.373 73.66) (width 0.254) (layer F.Cu) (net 6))
 (segment (start 158.373 73.66) (end 158.373 85.387) (width 0.254) (layer F.Cu) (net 6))
 (segment (start 158.373 85.387) (end 155.702 88.058) (width 0.254) (layer F.Cu) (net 6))
 (segment (start 161.544 78.66) (end 158.338 81.8659) (width 0.254) (layer B.Cu) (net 21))
 (segment (start 158.338 81.8659) (end 158.338 98.3548) (width 0.254) (layer B.Cu) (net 21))
 (segment (start 158.338 98.3548) (end 155.192 101.5) (width 0.254) (layer B.Cu) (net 21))
 (segment (start 155.192 101.5) (end 146.065 101.5) (width 0.254) (layer B.Cu) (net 21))
 (segment (start 146.065 101.5) (end 145.263 100.698) (width 0.254) (layer B.Cu) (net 21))
 (segment (start 145.263 100.698) (end 145.263 100.076) (width 0.254) (layer B.Cu) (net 21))
 (segment (start 145.263 100.076) (end 144.018 100.076) (width 0.254) (layer B.Cu) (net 21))
 (segment (start 151.892 78.74) (end 150.811 78.74) (width 0.254) (layer F.Cu) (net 9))
 (segment (start 150.811 78.74) (end 150.811 78.964) (width 0.254) (layer F.Cu) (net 9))
 (segment (start 150.811 78.964) (end 149.413 80.3613) (width 0.254) (layer F.Cu) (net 9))
 (segment (start 149.413 80.3613) (end 147.556 80.3613) (width 0.254) (layer F.Cu) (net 9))
 (segment (start 147.556 80.3613) (end 146.469 81.4485) (width 0.254) (layer F.Cu) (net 9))
 (segment (start 146.469 81.4485) (end 146.469 81.788) (width 0.254) (layer F.Cu) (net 9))
 (segment (start 146.469 81.788) (end 145.288 81.788) (width 0.254) (layer F.Cu) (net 9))
 (segment (start 155.702 83.058) (end 154.621 83.058) (width 0.254) (layer B.Cu) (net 9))
 (segment (start 154.621 83.058) (end 154.621 82.55) (width 0.254) (layer B.Cu) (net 9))
 (segment (start 154.621 82.55) (end 151.892 79.8213) (width 0.254) (layer B.Cu) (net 9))
 (segment (start 151.892 79.8213) (end 151.892 78.74) (width 0.254) (layer B.Cu) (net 9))
 (segment (start 146.558 100.076) (end 143.708 97.226) (width 0.254) (layer B.Cu) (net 11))
 (segment (start 143.708 97.226) (end 141.148 97.226) (width 0.254) (layer B.Cu) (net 11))
 (segment (start 141.148 97.226) (end 133.523 89.6009) (width 0.254) (layer B.Cu) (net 11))
 (segment (start 133.523 89.6009) (end 133.523 80.4367) (width 0.254) (layer B.Cu) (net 11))
 (segment (start 133.523 80.4367) (end 132.08 78.994) (width 0.254) (layer B.Cu) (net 11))
 (segment (start 135.89 99.822) (end 135.89 98.7407) (width 0.254) (layer B.Cu) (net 18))
 (segment (start 135.89 98.7407) (end 135.571 98.7407) (width 0.254) (layer B.Cu) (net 18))
 (segment (start 135.571 98.7407) (end 134.112 97.282) (width 0.254) (layer B.Cu) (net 18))
 (segment (start 141.478 69.85) (end 141.478 71.2473) (width 0.254) (layer B.Cu) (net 17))
 (segment (start 141.478 71.2473) (end 140.649 72.0761) (width 0.254) (layer B.Cu) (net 17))
 (segment (start 140.649 72.0761) (end 140.649 80.1395) (width 0.254) (layer B.Cu) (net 17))
 (segment (start 140.649 80.1395) (end 141.478 80.9683) (width 0.254) (layer B.Cu) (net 17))
 (segment (start 141.478 80.9683) (end 141.478 82.4673) (width 0.254) (layer B.Cu) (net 17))
 (segment (start 141.478 82.4673) (end 147.828 88.8173) (width 0.254) (layer B.Cu) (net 17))
 (segment (start 150.368 89.408) (end 151.549 89.408) (width 0.254) (layer F.Cu) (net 17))
 (segment (start 151.549 89.408) (end 154.343 92.202) (width 0.254) (layer F.Cu) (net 17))
 (segment (start 154.343 92.202) (end 155.448 92.202) (width 0.254) (layer F.Cu) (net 17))
 (segment (start 155.448 92.202) (end 156.529 92.202) (width 0.254) (layer F.Cu) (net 17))
 (segment (start 156.529 92.202) (end 156.529 91.8174) (width 0.254) (layer F.Cu) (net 17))
 (segment (start 156.529 91.8174) (end 160.209 88.138) (width 0.254) (layer F.Cu) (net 17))
 (segment (start 160.209 88.138) (end 161.29 88.138) (width 0.254) (layer F.Cu) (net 17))
 (segment (start 150.368 89.408) (end 149.187 89.408) (width 0.254) (layer B.Cu) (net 17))
 (segment (start 149.187 89.408) (end 148.596 88.8173) (width 0.254) (layer B.Cu) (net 17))
 (segment (start 148.596 88.8173) (end 147.828 88.8173) (width 0.254) (layer B.Cu) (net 17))
 (segment (start 147.828 89.408) (end 147.828 88.8173) (width 0.254) (layer B.Cu) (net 17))
 (segment (start 136.144 78.74) (end 136.144 77.6587) (width 0.254) (layer B.Cu) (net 1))
 (segment (start 136.144 77.6587) (end 137.225 76.5774) (width 0.254) (layer B.Cu) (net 1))
 (segment (start 137.225 76.5774) (end 137.225 69.6497) (width 0.254) (layer B.Cu) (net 1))
 (segment (start 137.225 69.6497) (end 138.432 68.4425) (width 0.254) (layer B.Cu) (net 1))
 (segment (start 138.432 68.4425) (end 144.528 68.4425) (width 0.254) (layer B.Cu) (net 1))
 (segment (start 144.528 68.4425) (end 145.313 69.2276) (width 0.254) (layer B.Cu) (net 1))
 (segment (start 145.313 69.2276) (end 145.313 69.85) (width 0.254) (layer B.Cu) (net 1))
 (segment (start 145.313 69.85) (end 146.558 69.85) (width 0.254) (layer B.Cu) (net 1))
 (segment (start 131.064 82.804) (end 132.145 82.804) (width 0.254) (layer F.Cu) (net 1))
 (segment (start 132.145 82.804) (end 133.161 81.788) (width 0.254) (layer F.Cu) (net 1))
 (segment (start 133.161 81.788) (end 135.128 81.788) (width 0.254) (layer F.Cu) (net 1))
 (segment (start 137.668 81.788) (end 135.128 81.788) (width 0.254) (layer F.Cu) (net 1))
 (segment (start 136.144 78.74) (end 136.144 79.8213) (width 0.254) (layer B.Cu) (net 1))
 (segment (start 136.144 79.8213) (end 135.913 79.8213) (width 0.254) (layer B.Cu) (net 1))
 (segment (start 135.913 79.8213) (end 135.128 80.6067) (width 0.254) (layer B.Cu) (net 1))
 (segment (start 135.128 80.6067) (end 135.128 81.788) (width 0.254) (layer B.Cu) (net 1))
 (segment (start 157.226 78.74) (end 156.145 78.74) (width 0.254) (layer F.Cu) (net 7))
 (segment (start 156.145 78.74) (end 156.145 78.852) (width 0.254) (layer F.Cu) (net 7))
 (segment (start 156.145 78.852) (end 153.209 81.788) (width 0.254) (layer F.Cu) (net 7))
 (segment (start 153.209 81.788) (end 150.368 81.788) (width 0.254) (layer F.Cu) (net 7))
 (segment (start 147.828 81.788) (end 150.368 81.788) (width 0.254) (layer F.Cu) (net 7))
 (segment (start 147.828 81.788) (end 147.828 80.6067) (width 0.254) (layer B.Cu) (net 7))
 (segment (start 147.828 80.6067) (end 147.339 80.1173) (width 0.254) (layer B.Cu) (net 7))
 (segment (start 147.339 80.1173) (end 147.339 73.1706) (width 0.254) (layer B.Cu) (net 7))
 (segment (start 147.339 73.1706) (end 144.018 69.85) (width 0.254) (layer B.Cu) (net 7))
 (segment (start 137.668 89.408) (end 137.668 88.2267) (width 0.254) (layer B.Cu) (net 14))
 (segment (start 137.668 88.2267) (end 138.938 86.9567) (width 0.254) (layer B.Cu) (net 14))
 (segment (start 138.938 86.9567) (end 138.938 69.85) (width 0.254) (layer B.Cu) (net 14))
 (segment (start 135.128 89.408) (end 133.947 89.408) (width 0.254) (layer F.Cu) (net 14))
 (segment (start 133.947 89.408) (end 133.947 90.4006) (width 0.254) (layer F.Cu) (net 14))
 (segment (start 133.947 90.4006) (end 132.145 92.202) (width 0.254) (layer F.Cu) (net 14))
 (segment (start 132.145 92.202) (end 131.064 92.202) (width 0.254) (layer F.Cu) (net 14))
 (segment (start 137.668 89.408) (end 135.128 89.408) (width 0.254) (layer F.Cu) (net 14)))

